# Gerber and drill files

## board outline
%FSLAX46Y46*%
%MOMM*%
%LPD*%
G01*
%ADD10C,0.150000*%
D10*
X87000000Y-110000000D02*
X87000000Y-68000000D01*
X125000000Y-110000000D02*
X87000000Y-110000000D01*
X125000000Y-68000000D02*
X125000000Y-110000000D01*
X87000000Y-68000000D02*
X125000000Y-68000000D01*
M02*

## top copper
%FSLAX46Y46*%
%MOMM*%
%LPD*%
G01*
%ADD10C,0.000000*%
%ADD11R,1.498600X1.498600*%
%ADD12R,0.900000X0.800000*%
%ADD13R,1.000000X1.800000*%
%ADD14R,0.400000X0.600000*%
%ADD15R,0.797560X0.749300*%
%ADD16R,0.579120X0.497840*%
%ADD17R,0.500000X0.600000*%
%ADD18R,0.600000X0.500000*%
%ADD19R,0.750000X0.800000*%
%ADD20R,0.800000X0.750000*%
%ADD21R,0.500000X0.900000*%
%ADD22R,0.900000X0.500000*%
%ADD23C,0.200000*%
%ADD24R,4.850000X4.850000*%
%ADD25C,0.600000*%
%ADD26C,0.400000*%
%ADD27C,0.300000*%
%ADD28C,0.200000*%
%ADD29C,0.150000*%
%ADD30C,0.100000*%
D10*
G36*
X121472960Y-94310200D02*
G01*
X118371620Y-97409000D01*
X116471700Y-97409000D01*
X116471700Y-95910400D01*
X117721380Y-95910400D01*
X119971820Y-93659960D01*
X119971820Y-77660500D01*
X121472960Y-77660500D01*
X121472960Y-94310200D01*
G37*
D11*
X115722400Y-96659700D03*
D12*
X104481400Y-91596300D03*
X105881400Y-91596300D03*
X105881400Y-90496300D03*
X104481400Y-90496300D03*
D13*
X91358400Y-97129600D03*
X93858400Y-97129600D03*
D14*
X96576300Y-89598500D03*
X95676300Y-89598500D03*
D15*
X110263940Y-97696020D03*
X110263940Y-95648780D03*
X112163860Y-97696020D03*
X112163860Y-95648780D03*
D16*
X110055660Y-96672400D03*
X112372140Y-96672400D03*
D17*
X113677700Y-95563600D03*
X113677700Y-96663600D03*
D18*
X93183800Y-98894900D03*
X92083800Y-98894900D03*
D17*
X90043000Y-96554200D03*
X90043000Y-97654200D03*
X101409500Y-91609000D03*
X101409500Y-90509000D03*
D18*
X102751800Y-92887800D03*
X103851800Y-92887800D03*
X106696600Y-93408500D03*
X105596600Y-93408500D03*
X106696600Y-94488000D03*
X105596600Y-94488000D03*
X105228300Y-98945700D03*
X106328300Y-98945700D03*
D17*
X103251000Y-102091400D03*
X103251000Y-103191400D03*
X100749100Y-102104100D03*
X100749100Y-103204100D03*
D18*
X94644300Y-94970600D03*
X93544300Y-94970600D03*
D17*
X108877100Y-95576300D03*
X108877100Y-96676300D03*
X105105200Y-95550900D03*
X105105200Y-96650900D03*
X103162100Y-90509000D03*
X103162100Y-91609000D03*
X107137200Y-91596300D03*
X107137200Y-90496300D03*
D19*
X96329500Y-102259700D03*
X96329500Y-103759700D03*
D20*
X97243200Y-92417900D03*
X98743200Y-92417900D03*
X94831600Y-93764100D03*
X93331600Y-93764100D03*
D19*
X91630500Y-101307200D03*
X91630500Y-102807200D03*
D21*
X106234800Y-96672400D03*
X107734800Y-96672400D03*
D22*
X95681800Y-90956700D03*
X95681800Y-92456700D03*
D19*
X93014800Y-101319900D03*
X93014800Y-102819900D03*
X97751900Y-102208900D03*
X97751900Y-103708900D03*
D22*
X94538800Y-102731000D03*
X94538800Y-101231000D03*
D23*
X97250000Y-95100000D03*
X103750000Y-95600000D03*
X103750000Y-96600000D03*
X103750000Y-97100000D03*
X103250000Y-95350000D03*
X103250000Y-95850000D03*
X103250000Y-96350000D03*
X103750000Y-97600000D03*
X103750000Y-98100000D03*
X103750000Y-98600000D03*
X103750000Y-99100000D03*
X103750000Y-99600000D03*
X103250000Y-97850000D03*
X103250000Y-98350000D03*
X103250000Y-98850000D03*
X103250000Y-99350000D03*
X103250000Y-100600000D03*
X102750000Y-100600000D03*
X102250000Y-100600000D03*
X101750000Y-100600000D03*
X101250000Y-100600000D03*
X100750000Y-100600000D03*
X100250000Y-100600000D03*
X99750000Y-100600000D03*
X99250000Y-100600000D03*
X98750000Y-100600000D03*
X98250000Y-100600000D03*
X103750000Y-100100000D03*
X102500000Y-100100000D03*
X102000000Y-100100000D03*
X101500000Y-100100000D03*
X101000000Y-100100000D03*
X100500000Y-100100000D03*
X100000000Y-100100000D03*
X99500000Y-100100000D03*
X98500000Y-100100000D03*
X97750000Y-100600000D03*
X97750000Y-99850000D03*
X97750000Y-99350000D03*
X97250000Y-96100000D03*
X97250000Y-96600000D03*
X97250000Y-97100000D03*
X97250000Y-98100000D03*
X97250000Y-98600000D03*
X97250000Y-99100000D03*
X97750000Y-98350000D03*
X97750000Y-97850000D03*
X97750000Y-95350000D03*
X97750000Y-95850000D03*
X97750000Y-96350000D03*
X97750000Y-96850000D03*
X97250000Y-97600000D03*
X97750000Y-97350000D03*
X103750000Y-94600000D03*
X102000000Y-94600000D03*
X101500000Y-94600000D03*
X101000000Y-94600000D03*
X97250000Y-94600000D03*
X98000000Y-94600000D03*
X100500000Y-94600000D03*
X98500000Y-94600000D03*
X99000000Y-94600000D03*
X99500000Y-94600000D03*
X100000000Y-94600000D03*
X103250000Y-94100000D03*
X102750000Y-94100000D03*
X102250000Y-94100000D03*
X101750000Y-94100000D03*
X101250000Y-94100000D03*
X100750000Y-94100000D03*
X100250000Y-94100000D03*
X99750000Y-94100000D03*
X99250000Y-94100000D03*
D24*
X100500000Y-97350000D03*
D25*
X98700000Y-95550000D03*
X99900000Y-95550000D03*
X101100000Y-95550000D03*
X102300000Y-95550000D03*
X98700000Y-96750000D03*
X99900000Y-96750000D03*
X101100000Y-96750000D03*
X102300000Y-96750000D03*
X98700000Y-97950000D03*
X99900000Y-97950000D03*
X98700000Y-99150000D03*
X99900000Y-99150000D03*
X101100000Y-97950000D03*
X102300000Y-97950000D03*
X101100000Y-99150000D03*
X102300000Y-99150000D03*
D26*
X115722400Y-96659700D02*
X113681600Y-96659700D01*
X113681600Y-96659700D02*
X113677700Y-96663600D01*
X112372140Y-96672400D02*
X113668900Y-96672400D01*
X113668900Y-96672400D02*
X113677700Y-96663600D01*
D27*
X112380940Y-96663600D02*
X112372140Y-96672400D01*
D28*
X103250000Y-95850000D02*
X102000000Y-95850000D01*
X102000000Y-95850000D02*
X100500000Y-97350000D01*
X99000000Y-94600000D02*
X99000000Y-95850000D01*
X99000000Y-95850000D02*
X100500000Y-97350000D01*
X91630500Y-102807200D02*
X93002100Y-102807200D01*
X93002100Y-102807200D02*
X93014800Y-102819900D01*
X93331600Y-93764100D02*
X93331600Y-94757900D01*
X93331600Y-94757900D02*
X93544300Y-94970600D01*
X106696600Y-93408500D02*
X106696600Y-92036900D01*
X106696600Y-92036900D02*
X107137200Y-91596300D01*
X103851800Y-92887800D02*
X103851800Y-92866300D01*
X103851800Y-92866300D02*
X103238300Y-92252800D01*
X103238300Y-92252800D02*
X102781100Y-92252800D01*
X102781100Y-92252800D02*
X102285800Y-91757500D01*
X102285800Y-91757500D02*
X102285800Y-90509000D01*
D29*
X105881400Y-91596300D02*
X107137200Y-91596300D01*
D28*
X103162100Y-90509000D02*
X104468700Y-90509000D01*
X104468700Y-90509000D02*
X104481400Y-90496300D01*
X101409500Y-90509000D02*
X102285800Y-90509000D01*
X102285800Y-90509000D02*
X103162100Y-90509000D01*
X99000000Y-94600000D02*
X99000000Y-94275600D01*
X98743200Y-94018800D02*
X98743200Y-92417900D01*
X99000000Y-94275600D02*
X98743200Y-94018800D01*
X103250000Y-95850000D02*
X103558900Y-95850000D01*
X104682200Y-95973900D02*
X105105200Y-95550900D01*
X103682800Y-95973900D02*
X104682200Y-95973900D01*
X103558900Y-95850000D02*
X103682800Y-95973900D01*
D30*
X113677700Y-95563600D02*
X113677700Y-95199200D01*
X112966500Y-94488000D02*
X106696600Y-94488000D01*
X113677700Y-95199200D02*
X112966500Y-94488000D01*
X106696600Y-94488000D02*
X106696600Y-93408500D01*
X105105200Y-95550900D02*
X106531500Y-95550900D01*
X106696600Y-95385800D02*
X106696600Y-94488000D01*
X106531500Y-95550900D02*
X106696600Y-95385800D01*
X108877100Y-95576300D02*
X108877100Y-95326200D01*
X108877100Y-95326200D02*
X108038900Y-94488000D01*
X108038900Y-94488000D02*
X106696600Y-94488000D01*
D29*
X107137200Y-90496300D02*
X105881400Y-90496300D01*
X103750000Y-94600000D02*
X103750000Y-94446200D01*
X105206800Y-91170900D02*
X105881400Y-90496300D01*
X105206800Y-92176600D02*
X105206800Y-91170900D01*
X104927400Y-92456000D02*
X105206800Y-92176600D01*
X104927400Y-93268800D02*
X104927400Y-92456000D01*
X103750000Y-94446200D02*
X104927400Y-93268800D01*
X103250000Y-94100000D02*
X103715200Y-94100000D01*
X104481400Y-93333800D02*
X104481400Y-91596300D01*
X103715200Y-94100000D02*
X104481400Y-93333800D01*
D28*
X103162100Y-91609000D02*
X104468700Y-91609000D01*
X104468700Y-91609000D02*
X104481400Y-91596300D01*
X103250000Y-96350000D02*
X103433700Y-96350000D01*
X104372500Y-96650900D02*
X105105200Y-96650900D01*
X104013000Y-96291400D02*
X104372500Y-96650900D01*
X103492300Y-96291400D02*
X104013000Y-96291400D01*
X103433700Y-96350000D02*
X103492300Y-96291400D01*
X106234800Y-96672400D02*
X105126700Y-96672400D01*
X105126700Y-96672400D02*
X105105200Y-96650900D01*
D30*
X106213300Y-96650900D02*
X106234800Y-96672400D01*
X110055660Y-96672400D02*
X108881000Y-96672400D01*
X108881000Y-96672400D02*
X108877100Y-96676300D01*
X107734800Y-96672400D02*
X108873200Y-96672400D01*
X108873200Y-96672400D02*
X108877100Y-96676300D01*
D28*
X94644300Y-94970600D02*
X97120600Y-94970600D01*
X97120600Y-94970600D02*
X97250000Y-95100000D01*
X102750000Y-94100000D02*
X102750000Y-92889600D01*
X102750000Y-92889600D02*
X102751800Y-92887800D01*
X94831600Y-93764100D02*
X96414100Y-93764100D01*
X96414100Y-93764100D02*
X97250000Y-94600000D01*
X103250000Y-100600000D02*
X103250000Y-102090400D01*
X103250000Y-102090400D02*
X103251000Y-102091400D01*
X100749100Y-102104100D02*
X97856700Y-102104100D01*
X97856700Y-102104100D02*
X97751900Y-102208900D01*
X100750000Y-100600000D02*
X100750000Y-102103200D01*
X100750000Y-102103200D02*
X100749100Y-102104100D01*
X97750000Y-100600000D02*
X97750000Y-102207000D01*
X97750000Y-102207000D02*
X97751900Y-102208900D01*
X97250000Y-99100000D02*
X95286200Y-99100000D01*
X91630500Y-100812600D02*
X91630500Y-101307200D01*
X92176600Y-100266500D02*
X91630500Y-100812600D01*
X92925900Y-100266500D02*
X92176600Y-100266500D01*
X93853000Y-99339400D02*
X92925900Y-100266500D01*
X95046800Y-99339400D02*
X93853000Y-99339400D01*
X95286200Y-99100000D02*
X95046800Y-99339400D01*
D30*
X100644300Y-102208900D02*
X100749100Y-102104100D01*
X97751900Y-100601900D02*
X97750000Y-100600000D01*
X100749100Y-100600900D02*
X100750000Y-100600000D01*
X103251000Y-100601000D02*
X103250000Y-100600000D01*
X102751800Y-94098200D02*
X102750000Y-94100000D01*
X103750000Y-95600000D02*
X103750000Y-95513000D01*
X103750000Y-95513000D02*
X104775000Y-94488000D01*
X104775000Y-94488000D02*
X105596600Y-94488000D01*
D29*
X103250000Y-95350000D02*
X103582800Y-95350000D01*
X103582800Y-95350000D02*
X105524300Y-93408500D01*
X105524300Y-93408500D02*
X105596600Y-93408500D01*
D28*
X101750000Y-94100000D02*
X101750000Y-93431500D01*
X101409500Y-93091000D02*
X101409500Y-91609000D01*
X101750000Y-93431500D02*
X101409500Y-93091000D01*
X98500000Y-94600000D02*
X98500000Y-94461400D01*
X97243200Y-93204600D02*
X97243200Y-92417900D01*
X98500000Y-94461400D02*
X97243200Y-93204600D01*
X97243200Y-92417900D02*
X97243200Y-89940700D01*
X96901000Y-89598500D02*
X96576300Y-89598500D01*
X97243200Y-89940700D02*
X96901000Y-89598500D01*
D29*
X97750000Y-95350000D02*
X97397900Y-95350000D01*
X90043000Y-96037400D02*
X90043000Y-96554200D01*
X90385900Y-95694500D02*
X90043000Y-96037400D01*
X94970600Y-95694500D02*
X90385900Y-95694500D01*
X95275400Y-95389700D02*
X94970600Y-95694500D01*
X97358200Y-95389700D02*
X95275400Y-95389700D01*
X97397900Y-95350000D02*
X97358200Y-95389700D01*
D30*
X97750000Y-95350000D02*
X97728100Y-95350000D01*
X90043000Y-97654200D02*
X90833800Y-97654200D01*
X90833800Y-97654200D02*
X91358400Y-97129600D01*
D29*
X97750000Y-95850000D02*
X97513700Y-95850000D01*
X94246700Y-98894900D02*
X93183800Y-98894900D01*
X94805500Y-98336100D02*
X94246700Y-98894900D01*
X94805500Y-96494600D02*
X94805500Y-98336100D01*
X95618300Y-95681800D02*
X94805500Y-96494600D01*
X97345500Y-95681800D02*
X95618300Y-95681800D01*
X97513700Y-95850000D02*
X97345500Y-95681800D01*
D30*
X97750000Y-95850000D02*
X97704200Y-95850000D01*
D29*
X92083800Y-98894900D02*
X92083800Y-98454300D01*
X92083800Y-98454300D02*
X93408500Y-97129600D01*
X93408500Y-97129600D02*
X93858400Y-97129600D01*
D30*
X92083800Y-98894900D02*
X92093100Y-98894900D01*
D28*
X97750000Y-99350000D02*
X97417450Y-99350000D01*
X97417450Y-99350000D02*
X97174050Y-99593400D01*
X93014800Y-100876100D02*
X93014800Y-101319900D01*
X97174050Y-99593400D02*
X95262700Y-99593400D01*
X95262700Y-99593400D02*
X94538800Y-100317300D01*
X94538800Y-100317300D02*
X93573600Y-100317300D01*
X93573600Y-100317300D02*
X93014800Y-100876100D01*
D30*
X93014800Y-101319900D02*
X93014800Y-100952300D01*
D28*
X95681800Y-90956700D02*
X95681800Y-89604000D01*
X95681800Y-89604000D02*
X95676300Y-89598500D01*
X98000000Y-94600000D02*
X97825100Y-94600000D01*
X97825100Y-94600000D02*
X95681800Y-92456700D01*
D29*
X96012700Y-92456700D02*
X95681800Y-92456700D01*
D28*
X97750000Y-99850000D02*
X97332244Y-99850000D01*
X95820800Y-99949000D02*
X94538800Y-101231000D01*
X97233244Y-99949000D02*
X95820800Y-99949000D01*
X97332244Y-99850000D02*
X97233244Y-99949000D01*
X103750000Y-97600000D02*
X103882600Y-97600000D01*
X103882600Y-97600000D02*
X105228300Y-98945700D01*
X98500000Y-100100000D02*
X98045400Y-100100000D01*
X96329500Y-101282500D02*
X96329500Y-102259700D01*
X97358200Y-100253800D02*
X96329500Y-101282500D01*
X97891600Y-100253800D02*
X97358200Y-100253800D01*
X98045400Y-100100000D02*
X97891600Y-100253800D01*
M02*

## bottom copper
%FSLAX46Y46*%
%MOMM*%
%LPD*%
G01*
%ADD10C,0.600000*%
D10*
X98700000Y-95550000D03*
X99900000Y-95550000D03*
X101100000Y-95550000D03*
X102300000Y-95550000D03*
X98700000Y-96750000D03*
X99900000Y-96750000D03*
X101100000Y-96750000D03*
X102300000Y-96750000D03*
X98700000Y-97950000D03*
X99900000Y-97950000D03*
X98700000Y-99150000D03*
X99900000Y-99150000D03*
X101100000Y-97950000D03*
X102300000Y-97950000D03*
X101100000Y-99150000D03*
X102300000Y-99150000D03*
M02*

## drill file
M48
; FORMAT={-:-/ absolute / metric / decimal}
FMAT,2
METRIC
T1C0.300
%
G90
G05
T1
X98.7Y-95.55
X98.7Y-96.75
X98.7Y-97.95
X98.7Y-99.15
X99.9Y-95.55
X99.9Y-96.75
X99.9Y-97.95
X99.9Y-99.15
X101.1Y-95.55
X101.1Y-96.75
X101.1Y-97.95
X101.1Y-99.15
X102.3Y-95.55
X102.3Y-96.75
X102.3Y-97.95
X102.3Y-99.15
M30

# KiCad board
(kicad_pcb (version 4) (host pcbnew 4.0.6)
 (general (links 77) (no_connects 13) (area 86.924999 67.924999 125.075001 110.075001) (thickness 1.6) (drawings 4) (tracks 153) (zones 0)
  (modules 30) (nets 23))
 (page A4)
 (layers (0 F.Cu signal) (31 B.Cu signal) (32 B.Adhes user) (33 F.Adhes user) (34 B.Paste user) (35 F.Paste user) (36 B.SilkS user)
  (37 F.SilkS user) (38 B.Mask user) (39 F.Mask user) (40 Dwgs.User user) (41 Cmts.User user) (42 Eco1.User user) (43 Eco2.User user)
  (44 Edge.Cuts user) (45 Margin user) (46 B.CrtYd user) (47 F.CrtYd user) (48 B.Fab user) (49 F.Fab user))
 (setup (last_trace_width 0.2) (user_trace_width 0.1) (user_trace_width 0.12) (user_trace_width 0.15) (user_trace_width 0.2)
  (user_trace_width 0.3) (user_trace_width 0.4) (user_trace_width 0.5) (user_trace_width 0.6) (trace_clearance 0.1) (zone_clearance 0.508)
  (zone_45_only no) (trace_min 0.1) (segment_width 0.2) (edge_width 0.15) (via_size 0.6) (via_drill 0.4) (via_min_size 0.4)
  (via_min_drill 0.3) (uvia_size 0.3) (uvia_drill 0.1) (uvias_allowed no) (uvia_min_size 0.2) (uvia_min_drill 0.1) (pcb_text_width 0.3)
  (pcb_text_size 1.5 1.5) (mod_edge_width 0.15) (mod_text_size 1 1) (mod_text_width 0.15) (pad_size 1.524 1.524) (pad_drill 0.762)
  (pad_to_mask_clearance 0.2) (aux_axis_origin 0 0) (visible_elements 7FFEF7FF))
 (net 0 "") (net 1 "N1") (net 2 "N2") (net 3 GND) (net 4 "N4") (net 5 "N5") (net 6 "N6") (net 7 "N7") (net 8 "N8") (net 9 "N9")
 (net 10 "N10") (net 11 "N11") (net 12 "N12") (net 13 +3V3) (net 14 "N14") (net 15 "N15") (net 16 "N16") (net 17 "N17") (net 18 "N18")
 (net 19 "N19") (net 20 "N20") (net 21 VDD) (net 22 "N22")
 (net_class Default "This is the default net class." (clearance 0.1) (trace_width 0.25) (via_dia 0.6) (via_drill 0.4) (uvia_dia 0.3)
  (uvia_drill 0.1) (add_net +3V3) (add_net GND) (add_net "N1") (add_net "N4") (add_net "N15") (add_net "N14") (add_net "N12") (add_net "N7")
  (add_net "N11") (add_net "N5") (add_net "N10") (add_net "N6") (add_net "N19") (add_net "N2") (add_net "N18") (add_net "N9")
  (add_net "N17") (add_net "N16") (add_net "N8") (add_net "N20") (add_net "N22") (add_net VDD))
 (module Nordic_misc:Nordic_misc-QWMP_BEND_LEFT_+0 (layer F.Cu) (at 114.9731 96.6597)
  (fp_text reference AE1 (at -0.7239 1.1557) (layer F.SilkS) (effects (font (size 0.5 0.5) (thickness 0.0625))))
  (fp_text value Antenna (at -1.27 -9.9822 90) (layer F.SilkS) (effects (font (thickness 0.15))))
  (fp_poly
   (pts (xy 1.4986 -0.7493) (xy 2.74828 -0.7493) (xy 4.99872 -2.99974) (xy 4.99872 -18.9992) (xy 6.49986 -18.9992) (xy 6.49986 -2.3495)
    (xy 3.39852 0.7493) (xy 1.4986 0.7493) (xy 1.4986 -0.7493))
   (layer F.Cu) (width 0))
  (pad 1 smd rect (at 0.7493 0) (size 1.4986 1.4986) (layers F.Cu F.Paste F.Mask) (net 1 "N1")))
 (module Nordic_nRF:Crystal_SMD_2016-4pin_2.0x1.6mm (layer F.Cu) (at 105.1814 91.0463)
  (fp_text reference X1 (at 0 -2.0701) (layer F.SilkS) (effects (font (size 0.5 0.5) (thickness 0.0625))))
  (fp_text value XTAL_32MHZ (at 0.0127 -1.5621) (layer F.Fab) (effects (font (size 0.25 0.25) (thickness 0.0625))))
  (pad 1 smd rect (at -0.7 0.55) (size 0.9 0.8) (layers F.Cu F.Paste F.Mask) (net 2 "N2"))
  (pad 2 smd rect (at 0.7 0.55) (size 0.9 0.8) (layers F.Cu F.Paste F.Mask) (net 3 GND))
  (pad 3 smd rect (at 0.7 -0.55) (size 0.9 0.8) (layers F.Cu F.Paste F.Mask) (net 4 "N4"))
  (pad 4 smd rect (at -0.7 -0.55) (size 0.9 0.8) (layers F.Cu F.Paste F.Mask) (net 3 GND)))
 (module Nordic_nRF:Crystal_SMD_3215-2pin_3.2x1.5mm (layer F.Cu) (at 92.6084 97.1296 180)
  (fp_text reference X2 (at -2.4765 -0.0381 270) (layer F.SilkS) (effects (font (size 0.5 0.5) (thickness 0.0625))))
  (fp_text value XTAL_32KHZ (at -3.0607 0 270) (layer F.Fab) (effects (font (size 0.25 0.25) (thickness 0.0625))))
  (pad 1 smd rect (at 1.25 0 180) (size 1 1.8) (layers F.Cu F.Paste F.Mask) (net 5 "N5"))
  (pad 2 smd rect (at -1.25 0 180) (size 1 1.8) (layers F.Cu F.Paste F.Mask) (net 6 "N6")))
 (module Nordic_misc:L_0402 (layer F.Cu) (at 96.1263 89.5985 180)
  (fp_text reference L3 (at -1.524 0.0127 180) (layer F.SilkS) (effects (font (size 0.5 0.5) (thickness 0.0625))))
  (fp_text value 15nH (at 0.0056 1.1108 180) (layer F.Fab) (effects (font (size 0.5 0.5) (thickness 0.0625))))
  (pad 1 smd rect (at -0.45 0 180) (size 0.4 0.6) (layers F.Cu F.Paste F.Mask) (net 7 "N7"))
  (pad 2 smd rect (at 0.45 0 180) (size 0.4 0.6) (layers F.Cu F.Paste F.Mask) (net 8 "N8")))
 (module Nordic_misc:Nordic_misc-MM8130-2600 (layer F.Cu) (at 111.2139 96.6724 90)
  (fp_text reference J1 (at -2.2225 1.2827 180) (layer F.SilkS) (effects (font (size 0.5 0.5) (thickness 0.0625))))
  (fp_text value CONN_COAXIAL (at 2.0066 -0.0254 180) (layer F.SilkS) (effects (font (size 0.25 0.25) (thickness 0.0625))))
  (pad 0 smd rect (at -1.02362 -0.94996 90) (size 0.7493 0.79756) (layers F.Cu F.Paste F.Mask))
  (pad 0 smd rect (at 1.02362 -0.94996 90) (size 0.7493 0.79756) (layers F.Cu F.Paste F.Mask))
  (pad 0 smd rect (at -1.02362 0.94996 90) (size 0.7493 0.79756) (layers F.Cu F.Paste F.Mask))
  (pad 0 smd rect (at 1.02362 0.94996 90) (size 0.7493 0.79756) (layers F.Cu F.Paste F.Mask))
  (pad 1 smd rect (at 0 -1.15824 90) (size 0.49784 0.57912) (layers F.Cu F.Paste F.Mask) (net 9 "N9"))
  (pad 2 smd rect (at 0 1.15824 90) (size 0.49784 0.57912) (layers F.Cu F.Paste F.Mask) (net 1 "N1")))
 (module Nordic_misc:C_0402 (layer F.Cu) (at 113.6777 96.1136 270)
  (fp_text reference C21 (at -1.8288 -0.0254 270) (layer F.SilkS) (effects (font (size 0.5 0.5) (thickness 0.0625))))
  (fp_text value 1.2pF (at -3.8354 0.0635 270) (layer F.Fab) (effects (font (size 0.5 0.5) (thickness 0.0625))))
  (pad 1 smd rect (at -0.55 0 270) (size 0.6 0.5) (layers F.Cu F.Paste F.Mask) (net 3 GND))
  (pad 2 smd rect (at 0.55 0 270) (size 0.6 0.5) (layers F.Cu F.Paste F.Mask) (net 1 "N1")))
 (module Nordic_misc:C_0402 (layer F.Cu) (at 92.6338 98.8949 180)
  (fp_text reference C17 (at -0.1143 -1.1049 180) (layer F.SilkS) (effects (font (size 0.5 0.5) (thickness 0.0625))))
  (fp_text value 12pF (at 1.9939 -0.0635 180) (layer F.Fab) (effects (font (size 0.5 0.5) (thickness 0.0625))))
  (pad 1 smd rect (at -0.55 0 180) (size 0.6 0.5) (layers F.Cu F.Paste F.Mask) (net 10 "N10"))
  (pad 2 smd rect (at 0.55 0 180) (size 0.6 0.5) (layers F.Cu F.Paste F.Mask) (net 6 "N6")))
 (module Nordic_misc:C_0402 (layer F.Cu) (at 90.043 97.1042 270)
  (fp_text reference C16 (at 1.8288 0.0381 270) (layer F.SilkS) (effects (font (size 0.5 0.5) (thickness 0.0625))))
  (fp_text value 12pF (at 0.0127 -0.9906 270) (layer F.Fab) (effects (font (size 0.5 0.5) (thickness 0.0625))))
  (pad 1 smd rect (at -0.55 0 270) (size 0.6 0.5) (layers F.Cu F.Paste F.Mask) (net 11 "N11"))
  (pad 2 smd rect (at 0.55 0 270) (size 0.6 0.5) (layers F.Cu F.Paste F.Mask) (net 5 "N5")))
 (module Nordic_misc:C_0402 (layer F.Cu) (at 101.4095 91.059 90)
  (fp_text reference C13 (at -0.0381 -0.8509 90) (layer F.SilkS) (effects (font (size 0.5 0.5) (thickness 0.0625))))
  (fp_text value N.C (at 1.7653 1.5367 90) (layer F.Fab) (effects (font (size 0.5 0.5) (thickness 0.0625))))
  (pad 1 smd rect (at -0.55 0 90) (size 0.6 0.5) (layers F.Cu F.Paste F.Mask) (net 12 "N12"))
  (pad 2 smd rect (at 0.55 0 90) (size 0.6 0.5) (layers F.Cu F.Paste F.Mask) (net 3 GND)))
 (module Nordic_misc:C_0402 (layer F.Cu) (at 103.3018 92.8878)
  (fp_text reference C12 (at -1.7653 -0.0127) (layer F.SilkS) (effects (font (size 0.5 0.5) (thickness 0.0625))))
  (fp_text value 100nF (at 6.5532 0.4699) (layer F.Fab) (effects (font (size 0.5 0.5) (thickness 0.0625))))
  (pad 1 smd rect (at -0.55 0) (size 0.6 0.5) (layers F.Cu F.Paste F.Mask) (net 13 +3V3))
  (pad 2 smd rect (at 0.55 0) (size 0.6 0.5) (layers F.Cu F.Paste F.Mask) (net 3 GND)))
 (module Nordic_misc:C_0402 (layer F.Cu) (at 106.1466 93.4085 180)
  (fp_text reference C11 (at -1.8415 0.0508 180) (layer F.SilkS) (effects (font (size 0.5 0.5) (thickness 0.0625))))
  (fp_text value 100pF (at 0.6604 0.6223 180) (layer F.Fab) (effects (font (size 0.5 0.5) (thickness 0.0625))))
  (pad 1 smd rect (at -0.55 0 180) (size 0.6 0.5) (layers F.Cu F.Paste F.Mask) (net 3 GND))
  (pad 2 smd rect (at 0.55 0 180) (size 0.6 0.5) (layers F.Cu F.Paste F.Mask) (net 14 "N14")))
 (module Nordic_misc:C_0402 (layer F.Cu) (at 106.1466 94.488 180)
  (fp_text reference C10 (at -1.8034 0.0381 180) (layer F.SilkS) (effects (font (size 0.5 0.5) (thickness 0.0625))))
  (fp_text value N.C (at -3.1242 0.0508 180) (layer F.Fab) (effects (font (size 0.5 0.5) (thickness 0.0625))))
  (pad 1 smd rect (at -0.55 0 180) (size 0.6 0.5) (layers F.Cu F.Paste F.Mask) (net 3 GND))
  (pad 2 smd rect (at 0.55 0 180) (size 0.6 0.5) (layers F.Cu F.Paste F.Mask) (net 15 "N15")))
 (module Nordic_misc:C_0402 (layer F.Cu) (at 105.7783 98.9457)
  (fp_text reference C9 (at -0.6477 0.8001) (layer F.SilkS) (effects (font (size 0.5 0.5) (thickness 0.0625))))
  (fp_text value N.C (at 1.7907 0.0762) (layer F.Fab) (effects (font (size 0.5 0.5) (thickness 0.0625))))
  (pad 1 smd rect (at -0.55 0) (size 0.6 0.5) (layers F.Cu F.Paste F.Mask) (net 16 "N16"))
  (pad 2 smd rect (at 0.55 0) (size 0.6 0.5) (layers F.Cu F.Paste F.Mask) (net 3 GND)))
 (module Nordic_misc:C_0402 (layer F.Cu) (at 103.251 102.6414 270)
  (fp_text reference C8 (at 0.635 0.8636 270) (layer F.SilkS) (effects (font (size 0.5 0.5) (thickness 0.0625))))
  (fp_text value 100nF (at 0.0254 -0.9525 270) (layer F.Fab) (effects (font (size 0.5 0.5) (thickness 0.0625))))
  (pad 1 smd rect (at -0.55 0 270) (size 0.6 0.5) (layers F.Cu F.Paste F.Mask) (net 13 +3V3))
  (pad 2 smd rect (at 0.55 0 270) (size 0.6 0.5) (layers F.Cu F.Paste F.Mask) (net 3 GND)))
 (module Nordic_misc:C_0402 (layer F.Cu) (at 100.7491 102.6541 270)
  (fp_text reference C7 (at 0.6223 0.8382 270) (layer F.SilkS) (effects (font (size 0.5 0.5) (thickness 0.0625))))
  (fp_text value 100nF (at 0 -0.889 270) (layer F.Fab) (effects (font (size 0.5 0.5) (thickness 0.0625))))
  (pad 1 smd rect (at -0.55 0 270) (size 0.6 0.5) (layers F.Cu F.Paste F.Mask) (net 13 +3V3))
  (pad 2 smd rect (at 0.55 0 270) (size 0.6 0.5) (layers F.Cu F.Paste F.Mask) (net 3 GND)))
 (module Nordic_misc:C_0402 (layer F.Cu) (at 94.0943 94.9706 180)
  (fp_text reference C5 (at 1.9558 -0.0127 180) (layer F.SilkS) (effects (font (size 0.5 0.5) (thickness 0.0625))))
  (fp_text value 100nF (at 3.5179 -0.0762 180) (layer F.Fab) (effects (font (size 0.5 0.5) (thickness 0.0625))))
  (pad 1 smd rect (at -0.55 0 180) (size 0.6 0.5) (layers F.Cu F.Paste F.Mask) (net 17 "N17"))
  (pad 2 smd rect (at 0.55 0 180) (size 0.6 0.5) (layers F.Cu F.Paste F.Mask) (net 3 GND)))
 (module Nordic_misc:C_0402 (layer F.Cu) (at 108.8771 96.1263 270)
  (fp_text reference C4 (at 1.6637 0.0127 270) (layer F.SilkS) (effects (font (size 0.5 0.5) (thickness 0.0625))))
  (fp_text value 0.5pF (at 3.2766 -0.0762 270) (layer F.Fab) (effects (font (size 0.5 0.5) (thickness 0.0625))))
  (pad 1 smd rect (at -0.55 0 270) (size 0.6 0.5) (layers F.Cu F.Paste F.Mask) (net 3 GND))
  (pad 2 smd rect (at 0.55 0 270) (size 0.6 0.5) (layers F.Cu F.Paste F.Mask) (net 9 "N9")))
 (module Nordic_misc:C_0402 (layer F.Cu) (at 105.1052 96.1009 270)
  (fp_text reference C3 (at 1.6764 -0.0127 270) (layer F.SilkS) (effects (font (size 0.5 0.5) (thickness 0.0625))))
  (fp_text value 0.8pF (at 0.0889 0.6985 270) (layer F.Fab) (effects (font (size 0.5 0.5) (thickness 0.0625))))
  (pad 1 smd rect (at -0.55 0 270) (size 0.6 0.5) (layers F.Cu F.Paste F.Mask) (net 3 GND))
  (pad 2 smd rect (at 0.55 0 270) (size 0.6 0.5) (layers F.Cu F.Paste F.Mask) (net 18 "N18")))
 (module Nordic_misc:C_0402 (layer F.Cu) (at 103.1621 91.059 270)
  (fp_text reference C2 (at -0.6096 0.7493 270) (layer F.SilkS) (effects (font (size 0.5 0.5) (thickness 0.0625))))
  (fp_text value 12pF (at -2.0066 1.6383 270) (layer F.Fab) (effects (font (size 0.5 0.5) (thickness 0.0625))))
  (pad 1 smd rect (at -0.55 0 270) (size 0.6 0.5) (layers F.Cu F.Paste F.Mask) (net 3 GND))
  (pad 2 smd rect (at 0.55 0 270) (size 0.6 0.5) (layers F.Cu F.Paste F.Mask) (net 2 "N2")))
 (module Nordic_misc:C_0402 (layer F.Cu) (at 107.1372 91.0463 90)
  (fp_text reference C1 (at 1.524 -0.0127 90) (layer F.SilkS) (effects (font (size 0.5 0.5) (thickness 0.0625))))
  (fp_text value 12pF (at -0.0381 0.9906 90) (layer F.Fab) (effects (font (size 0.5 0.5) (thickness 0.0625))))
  (pad 1 smd rect (at -0.55 0 90) (size 0.6 0.5) (layers F.Cu F.Paste F.Mask) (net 3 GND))
  (pad 2 smd rect (at 0.55 0 90) (size 0.6 0.5) (layers F.Cu F.Paste F.Mask) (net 4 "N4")))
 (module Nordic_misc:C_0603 (layer F.Cu) (at 96.3295 103.0097 270)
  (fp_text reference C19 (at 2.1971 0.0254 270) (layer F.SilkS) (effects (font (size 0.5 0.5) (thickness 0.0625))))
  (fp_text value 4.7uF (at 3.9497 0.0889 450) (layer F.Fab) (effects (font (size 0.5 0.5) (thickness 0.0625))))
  (pad 1 smd rect (at -0.75 0 270) (size 0.8 0.75) (layers F.Cu F.Paste F.Mask) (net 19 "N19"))
  (pad 2 smd rect (at 0.75 0 270) (size 0.8 0.75) (layers F.Cu F.Paste F.Mask) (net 3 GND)))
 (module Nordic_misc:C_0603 (layer F.Cu) (at 97.9932 92.4179)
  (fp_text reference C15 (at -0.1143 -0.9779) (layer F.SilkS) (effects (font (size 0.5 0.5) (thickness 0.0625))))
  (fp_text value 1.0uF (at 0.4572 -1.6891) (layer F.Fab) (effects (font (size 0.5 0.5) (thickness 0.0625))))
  (pad 1 smd rect (at -0.75 0) (size 0.8 0.75) (layers F.Cu F.Paste F.Mask) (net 7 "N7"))
  (pad 2 smd rect (at 0.75 0) (size 0.8 0.75) (layers F.Cu F.Paste F.Mask) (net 3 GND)))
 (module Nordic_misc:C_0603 (layer F.Cu) (at 94.0816 93.7641 180)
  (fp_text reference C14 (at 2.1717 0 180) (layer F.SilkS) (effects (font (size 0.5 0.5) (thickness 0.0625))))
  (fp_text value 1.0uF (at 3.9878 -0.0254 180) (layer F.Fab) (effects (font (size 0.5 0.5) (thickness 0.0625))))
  (pad 1 smd rect (at -0.75 0 180) (size 0.8 0.75) (layers F.Cu F.Paste F.Mask) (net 13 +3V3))
  (pad 2 smd rect (at 0.75 0 180) (size 0.8 0.75) (layers F.Cu F.Paste F.Mask) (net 3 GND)))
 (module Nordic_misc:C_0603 (layer F.Cu) (at 91.6305 102.0572 270)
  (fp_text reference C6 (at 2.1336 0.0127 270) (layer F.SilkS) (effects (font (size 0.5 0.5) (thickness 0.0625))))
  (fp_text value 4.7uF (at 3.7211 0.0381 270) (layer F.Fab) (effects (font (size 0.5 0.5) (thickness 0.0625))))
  (pad 1 smd rect (at -0.75 0 270) (size 0.8 0.75) (layers F.Cu F.Paste F.Mask) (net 13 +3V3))
  (pad 2 smd rect (at 0.75 0 270) (size 0.8 0.75) (layers F.Cu F.Paste F.Mask) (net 3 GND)))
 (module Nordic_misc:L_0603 (layer F.Cu) (at 106.9848 96.6724)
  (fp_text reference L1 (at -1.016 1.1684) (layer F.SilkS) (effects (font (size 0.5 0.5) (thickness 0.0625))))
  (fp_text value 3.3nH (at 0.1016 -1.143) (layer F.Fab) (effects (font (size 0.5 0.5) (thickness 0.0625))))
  (pad 1 smd rect (at -0.75 0) (size 0.5 0.9) (layers F.Cu F.Paste F.Mask) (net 18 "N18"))
  (pad 2 smd rect (at 0.75 0) (size 0.5 0.9) (layers F.Cu F.Paste F.Mask) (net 9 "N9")))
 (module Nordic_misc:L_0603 (layer F.Cu) (at 95.6818 91.7067 270)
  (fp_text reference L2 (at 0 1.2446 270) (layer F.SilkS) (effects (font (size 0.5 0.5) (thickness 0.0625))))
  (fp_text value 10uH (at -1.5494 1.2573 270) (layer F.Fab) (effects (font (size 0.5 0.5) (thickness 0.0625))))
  (pad 1 smd rect (at -0.75 0 270) (size 0.5 0.9) (layers F.Cu F.Paste F.Mask) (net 8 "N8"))
  (pad 2 smd rect (at 0.75 0 270) (size 0.5 0.9) (layers F.Cu F.Paste F.Mask) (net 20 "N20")))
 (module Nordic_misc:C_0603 (layer F.Cu) (at 93.0148 102.0699 270)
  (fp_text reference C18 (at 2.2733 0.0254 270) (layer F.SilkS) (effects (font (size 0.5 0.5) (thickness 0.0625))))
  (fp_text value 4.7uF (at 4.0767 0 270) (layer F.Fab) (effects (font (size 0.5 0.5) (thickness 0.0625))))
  (pad 1 smd rect (at -0.75 0 270) (size 0.8 0.75) (layers F.Cu F.Paste F.Mask) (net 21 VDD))
  (pad 2 smd rect (at 0.75 0 270) (size 0.8 0.75) (layers F.Cu F.Paste F.Mask) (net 3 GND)))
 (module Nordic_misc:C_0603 (layer F.Cu) (at 97.7519 102.9589 270)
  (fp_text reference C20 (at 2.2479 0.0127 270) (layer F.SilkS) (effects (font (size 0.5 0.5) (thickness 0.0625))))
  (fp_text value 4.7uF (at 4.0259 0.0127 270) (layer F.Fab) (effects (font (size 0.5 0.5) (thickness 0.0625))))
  (pad 1 smd rect (at -0.75 0 270) (size 0.8 0.75) (layers F.Cu F.Paste F.Mask) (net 13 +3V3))
  (pad 2 smd rect (at 0.75 0 270) (size 0.8 0.75) (layers F.Cu F.Paste F.Mask) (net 3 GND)))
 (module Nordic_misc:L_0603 (layer F.Cu) (at 94.5388 101.981 90)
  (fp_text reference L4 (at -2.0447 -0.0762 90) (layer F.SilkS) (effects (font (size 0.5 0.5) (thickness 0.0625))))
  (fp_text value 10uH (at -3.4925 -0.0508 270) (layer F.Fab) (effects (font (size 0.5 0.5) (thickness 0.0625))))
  (pad 1 smd rect (at -0.75 0 90) (size 0.5 0.9) (layers F.Cu F.Paste F.Mask) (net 13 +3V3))
  (pad 2 smd rect (at 0.75 0 90) (size 0.5 0.9) (layers F.Cu F.Paste F.Mask) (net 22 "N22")))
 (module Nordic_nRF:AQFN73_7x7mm (layer F.Cu) (at 100.5 97.35)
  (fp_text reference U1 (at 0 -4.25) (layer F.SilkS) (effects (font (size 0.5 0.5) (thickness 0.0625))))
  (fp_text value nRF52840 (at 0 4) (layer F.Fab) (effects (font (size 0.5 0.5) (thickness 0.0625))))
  (pad C1 smd circle (at -3.25 -2.25) (size 0.2 0.2) (layers F.Cu F.Paste F.Mask) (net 17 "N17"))
  (pad E24 smd circle (at 3.25 -1.75) (size 0.2 0.2) (layers F.Cu F.Paste F.Mask) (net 15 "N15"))
  (pad J24 smd circle (at 3.25 -0.75) (size 0.2 0.2) (layers F.Cu F.Paste F.Mask))
  (pad L24 smd circle (at 3.25 -0.25) (size 0.2 0.2) (layers F.Cu F.Paste F.Mask))
  (pad D23 smd circle (at 2.75 -2) (size 0.2 0.2) (layers F.Cu F.Paste F.Mask) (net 14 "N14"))
  (pad F23 smd circle (at 2.75 -1.5) (size 0.2 0.2) (layers F.Cu F.Paste F.Mask) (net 3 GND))
  (pad H23 smd circle (at 2.75 -1) (size 0.2 0.2) (layers F.Cu F.Paste F.Mask) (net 18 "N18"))
  (pad N24 smd circle (at 3.25 0.25) (size 0.2 0.2) (layers F.Cu F.Paste F.Mask) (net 16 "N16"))
  (pad R24 smd circle (at 3.25 0.75) (size 0.2 0.2) (layers F.Cu F.Paste F.Mask))
  (pad U24 smd circle (at 3.25 1.25) (size 0.2 0.2) (layers F.Cu F.Paste F.Mask))
  (pad W24 smd circle (at 3.25 1.75) (size 0.2 0.2) (layers F.Cu F.Paste F.Mask))
  (pad AA24 smd circle (at 3.25 2.25) (size 0.2 0.2) (layers F.Cu F.Paste F.Mask))
  (pad P23 smd circle (at 2.75 0.5) (size 0.2 0.2) (layers F.Cu F.Paste F.Mask))
  (pad T23 smd circle (at 2.75 1) (size 0.2 0.2) (layers F.Cu F.Paste F.Mask))
  (pad V23 smd circle (at 2.75 1.5) (size 0.2 0.2) (layers F.Cu F.Paste F.Mask))
  (pad Y23 smd circle (at 2.75 2) (size 0.2 0.2) (layers F.Cu F.Paste F.Mask))
  (pad AD23 smd circle (at 2.75 3.25) (size 0.2 0.2) (layers F.Cu F.Paste F.Mask) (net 13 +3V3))
  (pad AD22 smd circle (at 2.25 3.25) (size 0.2 0.2) (layers F.Cu F.Paste F.Mask))
  (pad AD20 smd circle (at 1.75 3.25) (size 0.2 0.2) (layers F.Cu F.Paste F.Mask))
  (pad AD18 smd circle (at 1.25 3.25) (size 0.2 0.2) (layers F.Cu F.Paste F.Mask))
  (pad AD16 smd circle (at 0.75 3.25) (size 0.2 0.2) (layers F.Cu F.Paste F.Mask))
  (pad AD14 smd circle (at 0.25 3.25) (size 0.2 0.2) (layers F.Cu F.Paste F.Mask) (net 13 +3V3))
  (pad AD12 smd circle (at -0.25 3.25) (size 0.2 0.2) (layers F.Cu F.Paste F.Mask))
  (pad AD10 smd circle (at -0.75 3.25) (size 0.2 0.2) (layers F.Cu F.Paste F.Mask))
  (pad AD8 smd circle (at -1.25 3.25) (size 0.2 0.2) (layers F.Cu F.Paste F.Mask))
  (pad AD6 smd circle (at -1.75 3.25) (size 0.2 0.2) (layers F.Cu F.Paste F.Mask))
  (pad AD4 smd circle (at -2.25 3.25) (size 0.2 0.2) (layers F.Cu F.Paste F.Mask))
  (pad AC24 smd circle (at 3.25 2.75) (size 0.2 0.2) (layers F.Cu F.Paste F.Mask))
  (pad AC21 smd circle (at 2 2.75) (size 0.2 0.2) (layers F.Cu F.Paste F.Mask))
  (pad AC19 smd circle (at 1.5 2.75) (size 0.2 0.2) (layers F.Cu F.Paste F.Mask))
  (pad AC17 smd circle (at 1 2.75) (size 0.2 0.2) (layers F.Cu F.Paste F.Mask))
  (pad AC15 smd circle (at 0.5 2.75) (size 0.2 0.2) (layers F.Cu F.Paste F.Mask))
  (pad AC13 smd circle (at 0 2.75) (size 0.2 0.2) (layers F.Cu F.Paste F.Mask))
  (pad AC11 smd circle (at -0.5 2.75) (size 0.2 0.2) (layers F.Cu F.Paste F.Mask))
  (pad AC9 smd circle (at -1 2.75) (size 0.2 0.2) (layers F.Cu F.Paste F.Mask))
  (pad AC5 smd circle (at -2 2.75) (size 0.2 0.2) (layers F.Cu F.Paste F.Mask) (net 19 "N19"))
  (pad AD2 smd circle (at -2.75 3.25) (size 0.2 0.2) (layers F.Cu F.Paste F.Mask) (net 13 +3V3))
  (pad AB2 smd circle (at -2.75 2.5) (size 0.2 0.2) (layers F.Cu F.Paste F.Mask) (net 22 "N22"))
  (pad Y2 smd circle (at -2.75 2) (size 0.2 0.2) (layers F.Cu F.Paste F.Mask) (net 21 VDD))
  (pad G1 smd circle (at -3.25 -1.25) (size 0.2 0.2) (layers F.Cu F.Paste F.Mask))
  (pad J1 smd circle (at -3.25 -0.75) (size 0.2 0.2) (layers F.Cu F.Paste F.Mask))
  (pad L1 smd circle (at -3.25 -0.25) (size 0.2 0.2) (layers F.Cu F.Paste F.Mask))
  (pad R1 smd circle (at -3.25 0.75) (size 0.2 0.2) (layers F.Cu F.Paste F.Mask))
  (pad U1 smd circle (at -3.25 1.25) (size 0.2 0.2) (layers F.Cu F.Paste F.Mask))
  (pad W1 smd circle (at -3.25 1.75) (size 0.2 0.2) (layers F.Cu F.Paste F.Mask) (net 13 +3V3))
  (pad T2 smd circle (at -2.75 1) (size 0.2 0.2) (layers F.Cu F.Paste F.Mask))
  (pad P2 smd circle (at -2.75 0.5) (size 0.2 0.2) (layers F.Cu F.Paste F.Mask))
  (pad D2 smd circle (at -2.75 -2) (size 0.2 0.2) (layers F.Cu F.Paste F.Mask) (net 11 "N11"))
  (pad F2 smd circle (at -2.75 -1.5) (size 0.2 0.2) (layers F.Cu F.Paste F.Mask) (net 10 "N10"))
  (pad H2 smd circle (at -2.75 -1) (size 0.2 0.2) (layers F.Cu F.Paste F.Mask))
  (pad K2 smd circle (at -2.75 -0.5) (size 0.2 0.2) (layers F.Cu F.Paste F.Mask))
  (pad N1 smd circle (at -3.25 0.25) (size 0.2 0.2) (layers F.Cu F.Paste F.Mask))
  (pad M2 smd circle (at -2.75 0) (size 0.2 0.2) (layers F.Cu F.Paste F.Mask))
  (pad B24 smd circle (at 3.25 -2.75) (size 0.2 0.2) (layers F.Cu F.Paste F.Mask) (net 4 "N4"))
  (pad B19 smd circle (at 1.5 -2.75) (size 0.2 0.2) (layers F.Cu F.Paste F.Mask))
  (pad B17 smd circle (at 1 -2.75) (size 0.2 0.2) (layers F.Cu F.Paste F.Mask))
  (pad B15 smd circle (at 0.5 -2.75) (size 0.2 0.2) (layers F.Cu F.Paste F.Mask))
  (pad B1 smd circle (at -3.25 -2.75) (size 0.2 0.2) (layers F.Cu F.Paste F.Mask) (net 13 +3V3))
  (pad B3 smd circle (at -2.5 -2.75) (size 0.2 0.2) (layers F.Cu F.Paste F.Mask) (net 20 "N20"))
  (pad B13 smd circle (at 0 -2.75) (size 0.2 0.2) (layers F.Cu F.Paste F.Mask))
  (pad B5 smd circle (at -2 -2.75) (size 0.2 0.2) (layers F.Cu F.Paste F.Mask) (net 7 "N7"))
  (pad B7 smd circle (at -1.5 -2.75) (size 0.2 0.2) (layers F.Cu F.Paste F.Mask) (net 3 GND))
  (pad B9 smd circle (at -1 -2.75) (size 0.2 0.2) (layers F.Cu F.Paste F.Mask))
  (pad B11 smd circle (at -0.5 -2.75) (size 0.2 0.2) (layers F.Cu F.Paste F.Mask))
  (pad A23 smd circle (at 2.75 -3.25) (size 0.2 0.2) (layers F.Cu F.Paste F.Mask) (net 2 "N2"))
  (pad A22 smd circle (at 2.25 -3.25) (size 0.2 0.2) (layers F.Cu F.Paste F.Mask) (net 13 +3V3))
  (pad A20 smd circle (at 1.75 -3.25) (size 0.2 0.2) (layers F.Cu F.Paste F.Mask))
  (pad A18 smd circle (at 1.25 -3.25) (size 0.2 0.2) (layers F.Cu F.Paste F.Mask) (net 12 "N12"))
  (pad A16 smd circle (at 0.75 -3.25) (size 0.2 0.2) (layers F.Cu F.Paste F.Mask))
  (pad A14 smd circle (at 0.25 -3.25) (size 0.2 0.2) (layers F.Cu F.Paste F.Mask))
  (pad A12 smd circle (at -0.25 -3.25) (size 0.2 0.2) (layers F.Cu F.Paste F.Mask))
  (pad A10 smd circle (at -0.75 -3.25) (size 0.2 0.2) (layers F.Cu F.Paste F.Mask))
  (pad A8 smd circle (at -1.25 -3.25) (size 0.2 0.2) (layers F.Cu F.Paste F.Mask))
  (pad 74 smd rect (at 0 0) (size 4.85 4.85) (layers F.Cu F.Paste F.Mask) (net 3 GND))
  (pad 74 thru_hole circle (at -1.8 -1.8) (size 0.6 0.6) (drill 0.3) (layers *.Cu) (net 3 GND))
  (pad 74 thru_hole circle (at -0.6 -1.8) (size 0.6 0.6) (drill 0.3) (layers *.Cu) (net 3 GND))
  (pad 74 thru_hole circle (at 0.6 -1.8) (size 0.6 0.6) (drill 0.3) (layers *.Cu) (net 3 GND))
  (pad 74 thru_hole circle (at 1.8 -1.8) (size 0.6 0.6) (drill 0.3) (layers *.Cu) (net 3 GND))
  (pad 74 thru_hole circle (at -1.8 -0.6) (size 0.6 0.6) (drill 0.3) (layers *.Cu) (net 3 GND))
  (pad 74 thru_hole circle (at -0.6 -0.6) (size 0.6 0.6) (drill 0.3) (layers *.Cu) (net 3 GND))
  (pad 74 thru_hole circle (at 0.6 -0.6) (size 0.6 0.6) (drill 0.3) (layers *.Cu) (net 3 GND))
  (pad 74 thru_hole circle (at 1.8 -0.6) (size 0.6 0.6) (drill 0.3) (layers *.Cu) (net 3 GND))
  (pad 74 thru_hole circle (at -1.8 0.6) (size 0.6 0.6) (drill 0.3) (layers *.Cu) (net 3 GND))
  (pad 74 thru_hole circle (at -0.6 0.6) (size 0.6 0.6) (drill 0.3) (layers *.Cu) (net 3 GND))
  (pad 74 thru_hole circle (at -1.8 1.8) (size 0.6 0.6) (drill 0.3) (layers *.Cu) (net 3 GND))
  (pad 74 thru_hole circle (at -0.6 1.8) (size 0.6 0.6) (drill 0.3) (layers *.Cu) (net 3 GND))
  (pad 74 thru_hole circle (at 0.6 0.6) (size 0.6 0.6) (drill 0.3) (layers *.Cu) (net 3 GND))
  (pad 74 thru_hole circle (at 1.8 0.6) (size 0.6 0.6) (drill 0.3) (layers *.Cu) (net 3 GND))
  (pad 74 thru_hole circle (at 0.6 1.8) (size 0.6 0.6) (drill 0.3) (layers *.Cu) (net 3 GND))
  (pad 74 thru_hole circle (at 1.8 1.8) (size 0.6 0.6) (drill 0.3) (layers *.Cu) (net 3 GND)))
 (gr_line (start 87 110) (end 87 68) (angle 90) (layer Edge.Cuts) (width 0.15))
 (gr_line (start 125 110) (end 87 110) (angle 90) (layer Edge.Cuts) (width 0.15))
 (gr_line (start 125 68) (end 125 110) (angle 90) (layer Edge.Cuts) (width 0.15))
 (gr_line (start 87 68) (end 125 68) (angle 90) (layer Edge.Cuts) (width 0.15))
 (segment (start 115.7224 96.6597) (end 113.6816 96.6597) (width 0.4) (layer F.Cu) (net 1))
 (segment (start 113.6816 96.6597) (end 113.6777 96.6636) (width 0.4) (layer F.Cu) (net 1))
 (segment (start 112.37214 96.6724) (end 113.6689 96.6724) (width 0.4) (layer F.Cu) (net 1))
 (segment (start 113.6689 96.6724) (end 113.6777 96.6636) (width 0.4) (layer F.Cu) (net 1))
 (segment (start 112.38094 96.6636) (end 112.37214 96.6724) (width 0.3) (layer F.Cu) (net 1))
 (segment (start 103.25 95.85) (end 102 95.85) (width 0.2) (layer F.Cu) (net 3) (status C00000))
 (segment (start 102 95.85) (end 100.5 97.35) (width 0.2) (layer F.Cu) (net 3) (status C00000))
 (segment (start 99 94.6) (end 99 95.85) (width 0.2) (layer F.Cu) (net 3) (status C00000))
 (segment (start 99 95.85) (end 100.5 97.35) (width 0.2) (layer F.Cu) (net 3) (status C00000))
 (segment (start 91.6305 102.8072) (end 93.0021 102.8072) (width 0.2) (layer F.Cu) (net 3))
 (segment (start 93.0021 102.8072) (end 93.0148 102.8199) (width 0.2) (layer F.Cu) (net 3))
 (segment (start 93.3316 93.7641) (end 93.3316 94.7579) (width 0.2) (layer F.Cu) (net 3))
 (segment (start 93.3316 94.7579) (end 93.5443 94.9706) (width 0.2) (layer F.Cu) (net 3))
 (segment (start 106.6966 93.4085) (end 106.6966 92.0369) (width 0.2) (layer F.Cu) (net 3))
 (segment (start 106.6966 92.0369) (end 107.1372 91.5963) (width 0.2) (layer F.Cu) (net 3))
 (segment (start 103.8518 92.8878) (end 103.8518 92.8663) (width 0.2) (layer F.Cu) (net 3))
 (segment (start 103.8518 92.8663) (end 103.2383 92.2528) (width 0.2) (layer F.Cu) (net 3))
 (segment (start 103.2383 92.2528) (end 102.7811 92.2528) (width 0.2) (layer F.Cu) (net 3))
 (segment (start 102.7811 92.2528) (end 102.2858 91.7575) (width 0.2) (layer F.Cu) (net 3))
 (segment (start 102.2858 91.7575) (end 102.2858 90.509) (width 0.2) (layer F.Cu) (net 3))
 (segment (start 105.8814 91.5963) (end 107.1372 91.5963) (width 0.15) (layer F.Cu) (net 3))
 (segment (start 103.1621 90.509) (end 104.4687 90.509) (width 0.2) (layer F.Cu) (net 3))
 (segment (start 104.4687 90.509) (end 104.4814 90.4963) (width 0.2) (layer F.Cu) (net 3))
 (segment (start 101.4095 90.509) (end 102.2858 90.509) (width 0.2) (layer F.Cu) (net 3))
 (segment (start 102.2858 90.509) (end 103.1621 90.509) (width 0.2) (layer F.Cu) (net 3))
 (segment (start 99 94.6) (end 99 94.2756) (width 0.2) (layer F.Cu) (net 3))
 (segment (start 98.7432 94.0188) (end 98.7432 92.4179) (width 0.2) (layer F.Cu) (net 3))
 (segment (start 99 94.2756) (end 98.7432 94.0188) (width 0.2) (layer F.Cu) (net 3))
 (segment (start 103.25 95.85) (end 103.5589 95.85) (width 0.2) (layer F.Cu) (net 3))
 (segment (start 104.6822 95.9739) (end 105.1052 95.5509) (width 0.2) (layer F.Cu) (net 3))
 (segment (start 103.6828 95.9739) (end 104.6822 95.9739) (width 0.2) (layer F.Cu) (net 3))
 (segment (start 103.5589 95.85) (end 103.6828 95.9739) (width 0.2) (layer F.Cu) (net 3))
 (segment (start 113.6777 95.5636) (end 113.6777 95.1992) (width 0.1) (layer F.Cu) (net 3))
 (segment (start 112.9665 94.488) (end 106.6966 94.488) (width 0.1) (layer F.Cu) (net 3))
 (segment (start 113.6777 95.1992) (end 112.9665 94.488) (width 0.1) (layer F.Cu) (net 3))
 (segment (start 106.6966 94.488) (end 106.6966 93.4085) (width 0.1) (layer F.Cu) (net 3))
 (segment (start 105.1052 95.5509) (end 106.5315 95.5509) (width 0.1) (layer F.Cu) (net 3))
 (segment (start 106.6966 95.3858) (end 106.6966 94.488) (width 0.1) (layer F.Cu) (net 3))
 (segment (start 106.5315 95.5509) (end 106.6966 95.3858) (width 0.1) (layer F.Cu) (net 3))
 (segment (start 108.8771 95.5763) (end 108.8771 95.3262) (width 0.1) (layer F.Cu) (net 3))
 (segment (start 108.8771 95.3262) (end 108.0389 94.488) (width 0.1) (layer F.Cu) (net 3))
 (segment (start 108.0389 94.488) (end 106.6966 94.488) (width 0.1) (layer F.Cu) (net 3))
 (segment (start 107.1372 90.4963) (end 105.8814 90.4963) (width 0.15) (layer F.Cu) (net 4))
 (segment (start 103.75 94.6) (end 103.75 94.4462) (width 0.15) (layer F.Cu) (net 4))
 (segment (start 105.2068 91.1709) (end 105.8814 90.4963) (width 0.15) (layer F.Cu) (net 4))
 (segment (start 105.2068 92.1766) (end 105.2068 91.1709) (width 0.15) (layer F.Cu) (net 4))
 (segment (start 104.9274 92.456) (end 105.2068 92.1766) (width 0.15) (layer F.Cu) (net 4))
 (segment (start 104.9274 93.2688) (end 104.9274 92.456) (width 0.15) (layer F.Cu) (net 4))
 (segment (start 103.75 94.4462) (end 104.9274 93.2688) (width 0.15) (layer F.Cu) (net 4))
 (segment (start 103.25 94.1) (end 103.7152 94.1) (width 0.15) (layer F.Cu) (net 2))
 (segment (start 104.4814 93.3338) (end 104.4814 91.5963) (width 0.15) (layer F.Cu) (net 2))
 (segment (start 103.7152 94.1) (end 104.4814 93.3338) (width 0.15) (layer F.Cu) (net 2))
 (segment (start 103.1621 91.609) (end 104.4687 91.609) (width 0.2) (layer F.Cu) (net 2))
 (segment (start 104.4687 91.609) (end 104.4814 91.5963) (width 0.2) (layer F.Cu) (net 2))
 (segment (start 103.25 96.35) (end 103.4337 96.35) (width 0.2) (layer F.Cu) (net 18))
 (segment (start 104.3725 96.6509) (end 105.1052 96.6509) (width 0.2) (layer F.Cu) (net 18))
 (segment (start 104.013 96.2914) (end 104.3725 96.6509) (width 0.2) (layer F.Cu) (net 18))
 (segment (start 103.4923 96.2914) (end 104.013 96.2914) (width 0.2) (layer F.Cu) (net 18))
 (segment (start 103.4337 96.35) (end 103.4923 96.2914) (width 0.2) (layer F.Cu) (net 18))
 (segment (start 106.2348 96.6724) (end 105.1267 96.6724) (width 0.2) (layer F.Cu) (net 18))
 (segment (start 105.1267 96.6724) (end 105.1052 96.6509) (width 0.2) (layer F.Cu) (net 18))
 (segment (start 106.2133 96.6509) (end 106.2348 96.6724) (width 0.1) (layer F.Cu) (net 18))
 (segment (start 110.05566 96.6724) (end 108.881 96.6724) (width 0.1) (layer F.Cu) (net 9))
 (segment (start 108.881 96.6724) (end 108.8771 96.6763) (width 0.1) (layer F.Cu) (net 9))
 (segment (start 107.7348 96.6724) (end 108.8732 96.6724) (width 0.1) (layer F.Cu) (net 9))
 (segment (start 108.8732 96.6724) (end 108.8771 96.6763) (width 0.1) (layer F.Cu) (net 9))
 (segment (start 94.6443 94.9706) (end 97.1206 94.9706) (width 0.2) (layer F.Cu) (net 17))
 (segment (start 97.1206 94.9706) (end 97.25 95.1) (width 0.2) (layer F.Cu) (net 17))
 (segment (start 102.75 94.1) (end 102.75 92.8896) (width 0.2) (layer F.Cu) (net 13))
 (segment (start 102.75 92.8896) (end 102.7518 92.8878) (width 0.2) (layer F.Cu) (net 13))
 (segment (start 94.8316 93.7641) (end 96.4141 93.7641) (width 0.2) (layer F.Cu) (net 13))
 (segment (start 96.4141 93.7641) (end 97.25 94.6) (width 0.2) (layer F.Cu) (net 13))
 (segment (start 103.25 100.6) (end 103.25 102.0904) (width 0.2) (layer F.Cu) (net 13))
 (segment (start 103.25 102.0904) (end 103.251 102.0914) (width 0.2) (layer F.Cu) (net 13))
 (segment (start 100.7491 102.1041) (end 97.8567 102.1041) (width 0.2) (layer F.Cu) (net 13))
 (segment (start 97.8567 102.1041) (end 97.7519 102.2089) (width 0.2) (layer F.Cu) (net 13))
 (segment (start 100.75 100.6) (end 100.75 102.1032) (width 0.2) (layer F.Cu) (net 13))
 (segment (start 100.75 102.1032) (end 100.7491 102.1041) (width 0.2) (layer F.Cu) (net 13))
 (segment (start 97.75 100.6) (end 97.75 102.207) (width 0.2) (layer F.Cu) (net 13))
 (segment (start 97.75 102.207) (end 97.7519 102.2089) (width 0.2) (layer F.Cu) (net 13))
 (segment (start 97.25 99.1) (end 95.2862 99.1) (width 0.2) (layer F.Cu) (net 13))
 (segment (start 91.6305 100.8126) (end 91.6305 101.3072) (width 0.2) (layer F.Cu) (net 13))
 (segment (start 92.1766 100.2665) (end 91.6305 100.8126) (width 0.2) (layer F.Cu) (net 13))
 (segment (start 92.9259 100.2665) (end 92.1766 100.2665) (width 0.2) (layer F.Cu) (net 13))
 (segment (start 93.853 99.3394) (end 92.9259 100.2665) (width 0.2) (layer F.Cu) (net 13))
 (segment (start 95.0468 99.3394) (end 93.853 99.3394) (width 0.2) (layer F.Cu) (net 13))
 (segment (start 95.2862 99.1) (end 95.0468 99.3394) (width 0.2) (layer F.Cu) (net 13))
 (segment (start 100.6443 102.2089) (end 100.7491 102.1041) (width 0.1) (layer F.Cu) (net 13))
 (segment (start 97.7519 100.6019) (end 97.75 100.6) (width 0.1) (layer F.Cu) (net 13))
 (segment (start 100.7491 100.6009) (end 100.75 100.6) (width 0.1) (layer F.Cu) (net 13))
 (segment (start 103.251 100.601) (end 103.25 100.6) (width 0.1) (layer F.Cu) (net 13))
 (segment (start 102.7518 94.0982) (end 102.75 94.1) (width 0.1) (layer F.Cu) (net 13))
 (segment (start 103.75 95.6) (end 103.75 95.513) (width 0.1) (layer F.Cu) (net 15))
 (segment (start 103.75 95.513) (end 104.775 94.488) (width 0.1) (layer F.Cu) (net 15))
 (segment (start 104.775 94.488) (end 105.5966 94.488) (width 0.1) (layer F.Cu) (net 15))
 (segment (start 103.25 95.35) (end 103.5828 95.35) (width 0.15) (layer F.Cu) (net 14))
 (segment (start 103.5828 95.35) (end 105.5243 93.4085) (width 0.15) (layer F.Cu) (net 14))
 (segment (start 105.5243 93.4085) (end 105.5966 93.4085) (width 0.15) (layer F.Cu) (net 14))
 (segment (start 101.75 94.1) (end 101.75 93.4315) (width 0.2) (layer F.Cu) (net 12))
 (segment (start 101.4095 93.091) (end 101.4095 91.609) (width 0.2) (layer F.Cu) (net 12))
 (segment (start 101.75 93.4315) (end 101.4095 93.091) (width 0.2) (layer F.Cu) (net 12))
 (segment (start 98.5 94.6) (end 98.5 94.4614) (width 0.2) (layer F.Cu) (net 7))
 (segment (start 97.2432 93.2046) (end 97.2432 92.4179) (width 0.2) (layer F.Cu) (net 7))
 (segment (start 98.5 94.4614) (end 97.2432 93.2046) (width 0.2) (layer F.Cu) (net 7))
 (segment (start 97.2432 92.4179) (end 97.2432 89.9407) (width 0.2) (layer F.Cu) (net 7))
 (segment (start 96.901 89.5985) (end 96.5763 89.5985) (width 0.2) (layer F.Cu) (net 7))
 (segment (start 97.2432 89.9407) (end 96.901 89.5985) (width 0.2) (layer F.Cu) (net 7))
 (segment (start 97.75 95.35) (end 97.3979 95.35) (width 0.15) (layer F.Cu) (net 11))
 (segment (start 90.043 96.0374) (end 90.043 96.5542) (width 0.15) (layer F.Cu) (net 11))
 (segment (start 90.3859 95.6945) (end 90.043 96.0374) (width 0.15) (layer F.Cu) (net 11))
 (segment (start 94.9706 95.6945) (end 90.3859 95.6945) (width 0.15) (layer F.Cu) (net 11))
 (segment (start 95.2754 95.3897) (end 94.9706 95.6945) (width 0.15) (layer F.Cu) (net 11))
 (segment (start 97.3582 95.3897) (end 95.2754 95.3897) (width 0.15) (layer F.Cu) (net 11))
 (segment (start 97.3979 95.35) (end 97.3582 95.3897) (width 0.15) (layer F.Cu) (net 11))
 (segment (start 97.75 95.35) (end 97.7281 95.35) (width 0.1) (layer F.Cu) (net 11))
 (segment (start 90.043 97.6542) (end 90.8338 97.6542) (width 0.1) (layer F.Cu) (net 5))
 (segment (start 90.8338 97.6542) (end 91.3584 97.1296) (width 0.1) (layer F.Cu) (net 5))
 (segment (start 97.75 95.85) (end 97.5137 95.85) (width 0.15) (layer F.Cu) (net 10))
 (segment (start 94.2467 98.8949) (end 93.1838 98.8949) (width 0.15) (layer F.Cu) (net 10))
 (segment (start 94.8055 98.3361) (end 94.2467 98.8949) (width 0.15) (layer F.Cu) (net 10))
 (segment (start 94.8055 96.4946) (end 94.8055 98.3361) (width 0.15) (layer F.Cu) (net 10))
 (segment (start 95.6183 95.6818) (end 94.8055 96.4946) (width 0.15) (layer F.Cu) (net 10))
 (segment (start 97.3455 95.6818) (end 95.6183 95.6818) (width 0.15) (layer F.Cu) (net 10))
 (segment (start 97.5137 95.85) (end 97.3455 95.6818) (width 0.15) (layer F.Cu) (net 10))
 (segment (start 97.75 95.85) (end 97.7042 95.85) (width 0.1) (layer F.Cu) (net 10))
 (segment (start 92.0838 98.8949) (end 92.0838 98.4543) (width 0.15) (layer F.Cu) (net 6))
 (segment (start 92.0838 98.4543) (end 93.4085 97.1296) (width 0.15) (layer F.Cu) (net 6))
 (segment (start 93.4085 97.1296) (end 93.8584 97.1296) (width 0.15) (layer F.Cu) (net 6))
 (segment (start 92.0838 98.8949) (end 92.0931 98.8949) (width 0.1) (layer F.Cu) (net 6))
 (segment (start 97.75 99.35) (end 97.41745 99.35) (width 0.2) (layer F.Cu) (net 21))
 (segment (start 97.41745 99.35) (end 97.17405 99.5934) (width 0.2) (layer F.Cu) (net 21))
 (segment (start 93.0148 100.8761) (end 93.0148 101.3199) (width 0.2) (layer F.Cu) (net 21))
 (segment (start 97.17405 99.5934) (end 95.2627 99.5934) (width 0.2) (layer F.Cu) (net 21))
 (segment (start 95.2627 99.5934) (end 94.5388 100.3173) (width 0.2) (layer F.Cu) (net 21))
 (segment (start 94.5388 100.3173) (end 93.5736 100.3173) (width 0.2) (layer F.Cu) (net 21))
 (segment (start 93.5736 100.3173) (end 93.0148 100.8761) (width 0.2) (layer F.Cu) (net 21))
 (segment (start 93.0148 101.3199) (end 93.0148 100.9523) (width 0.1) (layer F.Cu) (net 21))
 (segment (start 95.6818 90.9567) (end 95.6818 89.604) (width 0.2) (layer F.Cu) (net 8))
 (segment (start 95.6818 89.604) (end 95.6763 89.5985) (width 0.2) (layer F.Cu) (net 8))
 (segment (start 98 94.6) (end 97.8251 94.6) (width 0.2) (layer F.Cu) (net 20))
 (segment (start 97.8251 94.6) (end 95.6818 92.4567) (width 0.2) (layer F.Cu) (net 20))
 (segment (start 96.0127 92.4567) (end 95.6818 92.4567) (width 0.15) (layer F.Cu) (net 20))
 (segment (start 97.75 99.85) (end 97.332244 99.85) (width 0.2) (layer F.Cu) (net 22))
 (segment (start 95.8208 99.949) (end 94.5388 101.231) (width 0.2) (layer F.Cu) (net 22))
 (segment (start 97.233244 99.949) (end 95.8208 99.949) (width 0.2) (layer F.Cu) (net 22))
 (segment (start 97.332244 99.85) (end 97.233244 99.949) (width 0.2) (layer F.Cu) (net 22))
 (segment (start 103.75 97.6) (end 103.8826 97.6) (width 0.2) (layer F.Cu) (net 16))
 (segment (start 103.8826 97.6) (end 105.2283 98.9457) (width 0.2) (layer F.Cu) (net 16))
 (segment (start 98.5 100.1) (end 98.0454 100.1) (width 0.2) (layer F.Cu) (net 19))
 (segment (start 96.3295 101.2825) (end 96.3295 102.2597) (width 0.2) (layer F.Cu) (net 19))
 (segment (start 97.3582 100.2538) (end 96.3295 101.2825) (width 0.2) (layer F.Cu) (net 19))
 (segment (start 97.8916 100.2538) (end 97.3582 100.2538) (width 0.2) (layer F.Cu) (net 19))
 (segment (start 98.0454 100.1) (end 97.8916 100.2538) (width 0.2) (layer F.Cu) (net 19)))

